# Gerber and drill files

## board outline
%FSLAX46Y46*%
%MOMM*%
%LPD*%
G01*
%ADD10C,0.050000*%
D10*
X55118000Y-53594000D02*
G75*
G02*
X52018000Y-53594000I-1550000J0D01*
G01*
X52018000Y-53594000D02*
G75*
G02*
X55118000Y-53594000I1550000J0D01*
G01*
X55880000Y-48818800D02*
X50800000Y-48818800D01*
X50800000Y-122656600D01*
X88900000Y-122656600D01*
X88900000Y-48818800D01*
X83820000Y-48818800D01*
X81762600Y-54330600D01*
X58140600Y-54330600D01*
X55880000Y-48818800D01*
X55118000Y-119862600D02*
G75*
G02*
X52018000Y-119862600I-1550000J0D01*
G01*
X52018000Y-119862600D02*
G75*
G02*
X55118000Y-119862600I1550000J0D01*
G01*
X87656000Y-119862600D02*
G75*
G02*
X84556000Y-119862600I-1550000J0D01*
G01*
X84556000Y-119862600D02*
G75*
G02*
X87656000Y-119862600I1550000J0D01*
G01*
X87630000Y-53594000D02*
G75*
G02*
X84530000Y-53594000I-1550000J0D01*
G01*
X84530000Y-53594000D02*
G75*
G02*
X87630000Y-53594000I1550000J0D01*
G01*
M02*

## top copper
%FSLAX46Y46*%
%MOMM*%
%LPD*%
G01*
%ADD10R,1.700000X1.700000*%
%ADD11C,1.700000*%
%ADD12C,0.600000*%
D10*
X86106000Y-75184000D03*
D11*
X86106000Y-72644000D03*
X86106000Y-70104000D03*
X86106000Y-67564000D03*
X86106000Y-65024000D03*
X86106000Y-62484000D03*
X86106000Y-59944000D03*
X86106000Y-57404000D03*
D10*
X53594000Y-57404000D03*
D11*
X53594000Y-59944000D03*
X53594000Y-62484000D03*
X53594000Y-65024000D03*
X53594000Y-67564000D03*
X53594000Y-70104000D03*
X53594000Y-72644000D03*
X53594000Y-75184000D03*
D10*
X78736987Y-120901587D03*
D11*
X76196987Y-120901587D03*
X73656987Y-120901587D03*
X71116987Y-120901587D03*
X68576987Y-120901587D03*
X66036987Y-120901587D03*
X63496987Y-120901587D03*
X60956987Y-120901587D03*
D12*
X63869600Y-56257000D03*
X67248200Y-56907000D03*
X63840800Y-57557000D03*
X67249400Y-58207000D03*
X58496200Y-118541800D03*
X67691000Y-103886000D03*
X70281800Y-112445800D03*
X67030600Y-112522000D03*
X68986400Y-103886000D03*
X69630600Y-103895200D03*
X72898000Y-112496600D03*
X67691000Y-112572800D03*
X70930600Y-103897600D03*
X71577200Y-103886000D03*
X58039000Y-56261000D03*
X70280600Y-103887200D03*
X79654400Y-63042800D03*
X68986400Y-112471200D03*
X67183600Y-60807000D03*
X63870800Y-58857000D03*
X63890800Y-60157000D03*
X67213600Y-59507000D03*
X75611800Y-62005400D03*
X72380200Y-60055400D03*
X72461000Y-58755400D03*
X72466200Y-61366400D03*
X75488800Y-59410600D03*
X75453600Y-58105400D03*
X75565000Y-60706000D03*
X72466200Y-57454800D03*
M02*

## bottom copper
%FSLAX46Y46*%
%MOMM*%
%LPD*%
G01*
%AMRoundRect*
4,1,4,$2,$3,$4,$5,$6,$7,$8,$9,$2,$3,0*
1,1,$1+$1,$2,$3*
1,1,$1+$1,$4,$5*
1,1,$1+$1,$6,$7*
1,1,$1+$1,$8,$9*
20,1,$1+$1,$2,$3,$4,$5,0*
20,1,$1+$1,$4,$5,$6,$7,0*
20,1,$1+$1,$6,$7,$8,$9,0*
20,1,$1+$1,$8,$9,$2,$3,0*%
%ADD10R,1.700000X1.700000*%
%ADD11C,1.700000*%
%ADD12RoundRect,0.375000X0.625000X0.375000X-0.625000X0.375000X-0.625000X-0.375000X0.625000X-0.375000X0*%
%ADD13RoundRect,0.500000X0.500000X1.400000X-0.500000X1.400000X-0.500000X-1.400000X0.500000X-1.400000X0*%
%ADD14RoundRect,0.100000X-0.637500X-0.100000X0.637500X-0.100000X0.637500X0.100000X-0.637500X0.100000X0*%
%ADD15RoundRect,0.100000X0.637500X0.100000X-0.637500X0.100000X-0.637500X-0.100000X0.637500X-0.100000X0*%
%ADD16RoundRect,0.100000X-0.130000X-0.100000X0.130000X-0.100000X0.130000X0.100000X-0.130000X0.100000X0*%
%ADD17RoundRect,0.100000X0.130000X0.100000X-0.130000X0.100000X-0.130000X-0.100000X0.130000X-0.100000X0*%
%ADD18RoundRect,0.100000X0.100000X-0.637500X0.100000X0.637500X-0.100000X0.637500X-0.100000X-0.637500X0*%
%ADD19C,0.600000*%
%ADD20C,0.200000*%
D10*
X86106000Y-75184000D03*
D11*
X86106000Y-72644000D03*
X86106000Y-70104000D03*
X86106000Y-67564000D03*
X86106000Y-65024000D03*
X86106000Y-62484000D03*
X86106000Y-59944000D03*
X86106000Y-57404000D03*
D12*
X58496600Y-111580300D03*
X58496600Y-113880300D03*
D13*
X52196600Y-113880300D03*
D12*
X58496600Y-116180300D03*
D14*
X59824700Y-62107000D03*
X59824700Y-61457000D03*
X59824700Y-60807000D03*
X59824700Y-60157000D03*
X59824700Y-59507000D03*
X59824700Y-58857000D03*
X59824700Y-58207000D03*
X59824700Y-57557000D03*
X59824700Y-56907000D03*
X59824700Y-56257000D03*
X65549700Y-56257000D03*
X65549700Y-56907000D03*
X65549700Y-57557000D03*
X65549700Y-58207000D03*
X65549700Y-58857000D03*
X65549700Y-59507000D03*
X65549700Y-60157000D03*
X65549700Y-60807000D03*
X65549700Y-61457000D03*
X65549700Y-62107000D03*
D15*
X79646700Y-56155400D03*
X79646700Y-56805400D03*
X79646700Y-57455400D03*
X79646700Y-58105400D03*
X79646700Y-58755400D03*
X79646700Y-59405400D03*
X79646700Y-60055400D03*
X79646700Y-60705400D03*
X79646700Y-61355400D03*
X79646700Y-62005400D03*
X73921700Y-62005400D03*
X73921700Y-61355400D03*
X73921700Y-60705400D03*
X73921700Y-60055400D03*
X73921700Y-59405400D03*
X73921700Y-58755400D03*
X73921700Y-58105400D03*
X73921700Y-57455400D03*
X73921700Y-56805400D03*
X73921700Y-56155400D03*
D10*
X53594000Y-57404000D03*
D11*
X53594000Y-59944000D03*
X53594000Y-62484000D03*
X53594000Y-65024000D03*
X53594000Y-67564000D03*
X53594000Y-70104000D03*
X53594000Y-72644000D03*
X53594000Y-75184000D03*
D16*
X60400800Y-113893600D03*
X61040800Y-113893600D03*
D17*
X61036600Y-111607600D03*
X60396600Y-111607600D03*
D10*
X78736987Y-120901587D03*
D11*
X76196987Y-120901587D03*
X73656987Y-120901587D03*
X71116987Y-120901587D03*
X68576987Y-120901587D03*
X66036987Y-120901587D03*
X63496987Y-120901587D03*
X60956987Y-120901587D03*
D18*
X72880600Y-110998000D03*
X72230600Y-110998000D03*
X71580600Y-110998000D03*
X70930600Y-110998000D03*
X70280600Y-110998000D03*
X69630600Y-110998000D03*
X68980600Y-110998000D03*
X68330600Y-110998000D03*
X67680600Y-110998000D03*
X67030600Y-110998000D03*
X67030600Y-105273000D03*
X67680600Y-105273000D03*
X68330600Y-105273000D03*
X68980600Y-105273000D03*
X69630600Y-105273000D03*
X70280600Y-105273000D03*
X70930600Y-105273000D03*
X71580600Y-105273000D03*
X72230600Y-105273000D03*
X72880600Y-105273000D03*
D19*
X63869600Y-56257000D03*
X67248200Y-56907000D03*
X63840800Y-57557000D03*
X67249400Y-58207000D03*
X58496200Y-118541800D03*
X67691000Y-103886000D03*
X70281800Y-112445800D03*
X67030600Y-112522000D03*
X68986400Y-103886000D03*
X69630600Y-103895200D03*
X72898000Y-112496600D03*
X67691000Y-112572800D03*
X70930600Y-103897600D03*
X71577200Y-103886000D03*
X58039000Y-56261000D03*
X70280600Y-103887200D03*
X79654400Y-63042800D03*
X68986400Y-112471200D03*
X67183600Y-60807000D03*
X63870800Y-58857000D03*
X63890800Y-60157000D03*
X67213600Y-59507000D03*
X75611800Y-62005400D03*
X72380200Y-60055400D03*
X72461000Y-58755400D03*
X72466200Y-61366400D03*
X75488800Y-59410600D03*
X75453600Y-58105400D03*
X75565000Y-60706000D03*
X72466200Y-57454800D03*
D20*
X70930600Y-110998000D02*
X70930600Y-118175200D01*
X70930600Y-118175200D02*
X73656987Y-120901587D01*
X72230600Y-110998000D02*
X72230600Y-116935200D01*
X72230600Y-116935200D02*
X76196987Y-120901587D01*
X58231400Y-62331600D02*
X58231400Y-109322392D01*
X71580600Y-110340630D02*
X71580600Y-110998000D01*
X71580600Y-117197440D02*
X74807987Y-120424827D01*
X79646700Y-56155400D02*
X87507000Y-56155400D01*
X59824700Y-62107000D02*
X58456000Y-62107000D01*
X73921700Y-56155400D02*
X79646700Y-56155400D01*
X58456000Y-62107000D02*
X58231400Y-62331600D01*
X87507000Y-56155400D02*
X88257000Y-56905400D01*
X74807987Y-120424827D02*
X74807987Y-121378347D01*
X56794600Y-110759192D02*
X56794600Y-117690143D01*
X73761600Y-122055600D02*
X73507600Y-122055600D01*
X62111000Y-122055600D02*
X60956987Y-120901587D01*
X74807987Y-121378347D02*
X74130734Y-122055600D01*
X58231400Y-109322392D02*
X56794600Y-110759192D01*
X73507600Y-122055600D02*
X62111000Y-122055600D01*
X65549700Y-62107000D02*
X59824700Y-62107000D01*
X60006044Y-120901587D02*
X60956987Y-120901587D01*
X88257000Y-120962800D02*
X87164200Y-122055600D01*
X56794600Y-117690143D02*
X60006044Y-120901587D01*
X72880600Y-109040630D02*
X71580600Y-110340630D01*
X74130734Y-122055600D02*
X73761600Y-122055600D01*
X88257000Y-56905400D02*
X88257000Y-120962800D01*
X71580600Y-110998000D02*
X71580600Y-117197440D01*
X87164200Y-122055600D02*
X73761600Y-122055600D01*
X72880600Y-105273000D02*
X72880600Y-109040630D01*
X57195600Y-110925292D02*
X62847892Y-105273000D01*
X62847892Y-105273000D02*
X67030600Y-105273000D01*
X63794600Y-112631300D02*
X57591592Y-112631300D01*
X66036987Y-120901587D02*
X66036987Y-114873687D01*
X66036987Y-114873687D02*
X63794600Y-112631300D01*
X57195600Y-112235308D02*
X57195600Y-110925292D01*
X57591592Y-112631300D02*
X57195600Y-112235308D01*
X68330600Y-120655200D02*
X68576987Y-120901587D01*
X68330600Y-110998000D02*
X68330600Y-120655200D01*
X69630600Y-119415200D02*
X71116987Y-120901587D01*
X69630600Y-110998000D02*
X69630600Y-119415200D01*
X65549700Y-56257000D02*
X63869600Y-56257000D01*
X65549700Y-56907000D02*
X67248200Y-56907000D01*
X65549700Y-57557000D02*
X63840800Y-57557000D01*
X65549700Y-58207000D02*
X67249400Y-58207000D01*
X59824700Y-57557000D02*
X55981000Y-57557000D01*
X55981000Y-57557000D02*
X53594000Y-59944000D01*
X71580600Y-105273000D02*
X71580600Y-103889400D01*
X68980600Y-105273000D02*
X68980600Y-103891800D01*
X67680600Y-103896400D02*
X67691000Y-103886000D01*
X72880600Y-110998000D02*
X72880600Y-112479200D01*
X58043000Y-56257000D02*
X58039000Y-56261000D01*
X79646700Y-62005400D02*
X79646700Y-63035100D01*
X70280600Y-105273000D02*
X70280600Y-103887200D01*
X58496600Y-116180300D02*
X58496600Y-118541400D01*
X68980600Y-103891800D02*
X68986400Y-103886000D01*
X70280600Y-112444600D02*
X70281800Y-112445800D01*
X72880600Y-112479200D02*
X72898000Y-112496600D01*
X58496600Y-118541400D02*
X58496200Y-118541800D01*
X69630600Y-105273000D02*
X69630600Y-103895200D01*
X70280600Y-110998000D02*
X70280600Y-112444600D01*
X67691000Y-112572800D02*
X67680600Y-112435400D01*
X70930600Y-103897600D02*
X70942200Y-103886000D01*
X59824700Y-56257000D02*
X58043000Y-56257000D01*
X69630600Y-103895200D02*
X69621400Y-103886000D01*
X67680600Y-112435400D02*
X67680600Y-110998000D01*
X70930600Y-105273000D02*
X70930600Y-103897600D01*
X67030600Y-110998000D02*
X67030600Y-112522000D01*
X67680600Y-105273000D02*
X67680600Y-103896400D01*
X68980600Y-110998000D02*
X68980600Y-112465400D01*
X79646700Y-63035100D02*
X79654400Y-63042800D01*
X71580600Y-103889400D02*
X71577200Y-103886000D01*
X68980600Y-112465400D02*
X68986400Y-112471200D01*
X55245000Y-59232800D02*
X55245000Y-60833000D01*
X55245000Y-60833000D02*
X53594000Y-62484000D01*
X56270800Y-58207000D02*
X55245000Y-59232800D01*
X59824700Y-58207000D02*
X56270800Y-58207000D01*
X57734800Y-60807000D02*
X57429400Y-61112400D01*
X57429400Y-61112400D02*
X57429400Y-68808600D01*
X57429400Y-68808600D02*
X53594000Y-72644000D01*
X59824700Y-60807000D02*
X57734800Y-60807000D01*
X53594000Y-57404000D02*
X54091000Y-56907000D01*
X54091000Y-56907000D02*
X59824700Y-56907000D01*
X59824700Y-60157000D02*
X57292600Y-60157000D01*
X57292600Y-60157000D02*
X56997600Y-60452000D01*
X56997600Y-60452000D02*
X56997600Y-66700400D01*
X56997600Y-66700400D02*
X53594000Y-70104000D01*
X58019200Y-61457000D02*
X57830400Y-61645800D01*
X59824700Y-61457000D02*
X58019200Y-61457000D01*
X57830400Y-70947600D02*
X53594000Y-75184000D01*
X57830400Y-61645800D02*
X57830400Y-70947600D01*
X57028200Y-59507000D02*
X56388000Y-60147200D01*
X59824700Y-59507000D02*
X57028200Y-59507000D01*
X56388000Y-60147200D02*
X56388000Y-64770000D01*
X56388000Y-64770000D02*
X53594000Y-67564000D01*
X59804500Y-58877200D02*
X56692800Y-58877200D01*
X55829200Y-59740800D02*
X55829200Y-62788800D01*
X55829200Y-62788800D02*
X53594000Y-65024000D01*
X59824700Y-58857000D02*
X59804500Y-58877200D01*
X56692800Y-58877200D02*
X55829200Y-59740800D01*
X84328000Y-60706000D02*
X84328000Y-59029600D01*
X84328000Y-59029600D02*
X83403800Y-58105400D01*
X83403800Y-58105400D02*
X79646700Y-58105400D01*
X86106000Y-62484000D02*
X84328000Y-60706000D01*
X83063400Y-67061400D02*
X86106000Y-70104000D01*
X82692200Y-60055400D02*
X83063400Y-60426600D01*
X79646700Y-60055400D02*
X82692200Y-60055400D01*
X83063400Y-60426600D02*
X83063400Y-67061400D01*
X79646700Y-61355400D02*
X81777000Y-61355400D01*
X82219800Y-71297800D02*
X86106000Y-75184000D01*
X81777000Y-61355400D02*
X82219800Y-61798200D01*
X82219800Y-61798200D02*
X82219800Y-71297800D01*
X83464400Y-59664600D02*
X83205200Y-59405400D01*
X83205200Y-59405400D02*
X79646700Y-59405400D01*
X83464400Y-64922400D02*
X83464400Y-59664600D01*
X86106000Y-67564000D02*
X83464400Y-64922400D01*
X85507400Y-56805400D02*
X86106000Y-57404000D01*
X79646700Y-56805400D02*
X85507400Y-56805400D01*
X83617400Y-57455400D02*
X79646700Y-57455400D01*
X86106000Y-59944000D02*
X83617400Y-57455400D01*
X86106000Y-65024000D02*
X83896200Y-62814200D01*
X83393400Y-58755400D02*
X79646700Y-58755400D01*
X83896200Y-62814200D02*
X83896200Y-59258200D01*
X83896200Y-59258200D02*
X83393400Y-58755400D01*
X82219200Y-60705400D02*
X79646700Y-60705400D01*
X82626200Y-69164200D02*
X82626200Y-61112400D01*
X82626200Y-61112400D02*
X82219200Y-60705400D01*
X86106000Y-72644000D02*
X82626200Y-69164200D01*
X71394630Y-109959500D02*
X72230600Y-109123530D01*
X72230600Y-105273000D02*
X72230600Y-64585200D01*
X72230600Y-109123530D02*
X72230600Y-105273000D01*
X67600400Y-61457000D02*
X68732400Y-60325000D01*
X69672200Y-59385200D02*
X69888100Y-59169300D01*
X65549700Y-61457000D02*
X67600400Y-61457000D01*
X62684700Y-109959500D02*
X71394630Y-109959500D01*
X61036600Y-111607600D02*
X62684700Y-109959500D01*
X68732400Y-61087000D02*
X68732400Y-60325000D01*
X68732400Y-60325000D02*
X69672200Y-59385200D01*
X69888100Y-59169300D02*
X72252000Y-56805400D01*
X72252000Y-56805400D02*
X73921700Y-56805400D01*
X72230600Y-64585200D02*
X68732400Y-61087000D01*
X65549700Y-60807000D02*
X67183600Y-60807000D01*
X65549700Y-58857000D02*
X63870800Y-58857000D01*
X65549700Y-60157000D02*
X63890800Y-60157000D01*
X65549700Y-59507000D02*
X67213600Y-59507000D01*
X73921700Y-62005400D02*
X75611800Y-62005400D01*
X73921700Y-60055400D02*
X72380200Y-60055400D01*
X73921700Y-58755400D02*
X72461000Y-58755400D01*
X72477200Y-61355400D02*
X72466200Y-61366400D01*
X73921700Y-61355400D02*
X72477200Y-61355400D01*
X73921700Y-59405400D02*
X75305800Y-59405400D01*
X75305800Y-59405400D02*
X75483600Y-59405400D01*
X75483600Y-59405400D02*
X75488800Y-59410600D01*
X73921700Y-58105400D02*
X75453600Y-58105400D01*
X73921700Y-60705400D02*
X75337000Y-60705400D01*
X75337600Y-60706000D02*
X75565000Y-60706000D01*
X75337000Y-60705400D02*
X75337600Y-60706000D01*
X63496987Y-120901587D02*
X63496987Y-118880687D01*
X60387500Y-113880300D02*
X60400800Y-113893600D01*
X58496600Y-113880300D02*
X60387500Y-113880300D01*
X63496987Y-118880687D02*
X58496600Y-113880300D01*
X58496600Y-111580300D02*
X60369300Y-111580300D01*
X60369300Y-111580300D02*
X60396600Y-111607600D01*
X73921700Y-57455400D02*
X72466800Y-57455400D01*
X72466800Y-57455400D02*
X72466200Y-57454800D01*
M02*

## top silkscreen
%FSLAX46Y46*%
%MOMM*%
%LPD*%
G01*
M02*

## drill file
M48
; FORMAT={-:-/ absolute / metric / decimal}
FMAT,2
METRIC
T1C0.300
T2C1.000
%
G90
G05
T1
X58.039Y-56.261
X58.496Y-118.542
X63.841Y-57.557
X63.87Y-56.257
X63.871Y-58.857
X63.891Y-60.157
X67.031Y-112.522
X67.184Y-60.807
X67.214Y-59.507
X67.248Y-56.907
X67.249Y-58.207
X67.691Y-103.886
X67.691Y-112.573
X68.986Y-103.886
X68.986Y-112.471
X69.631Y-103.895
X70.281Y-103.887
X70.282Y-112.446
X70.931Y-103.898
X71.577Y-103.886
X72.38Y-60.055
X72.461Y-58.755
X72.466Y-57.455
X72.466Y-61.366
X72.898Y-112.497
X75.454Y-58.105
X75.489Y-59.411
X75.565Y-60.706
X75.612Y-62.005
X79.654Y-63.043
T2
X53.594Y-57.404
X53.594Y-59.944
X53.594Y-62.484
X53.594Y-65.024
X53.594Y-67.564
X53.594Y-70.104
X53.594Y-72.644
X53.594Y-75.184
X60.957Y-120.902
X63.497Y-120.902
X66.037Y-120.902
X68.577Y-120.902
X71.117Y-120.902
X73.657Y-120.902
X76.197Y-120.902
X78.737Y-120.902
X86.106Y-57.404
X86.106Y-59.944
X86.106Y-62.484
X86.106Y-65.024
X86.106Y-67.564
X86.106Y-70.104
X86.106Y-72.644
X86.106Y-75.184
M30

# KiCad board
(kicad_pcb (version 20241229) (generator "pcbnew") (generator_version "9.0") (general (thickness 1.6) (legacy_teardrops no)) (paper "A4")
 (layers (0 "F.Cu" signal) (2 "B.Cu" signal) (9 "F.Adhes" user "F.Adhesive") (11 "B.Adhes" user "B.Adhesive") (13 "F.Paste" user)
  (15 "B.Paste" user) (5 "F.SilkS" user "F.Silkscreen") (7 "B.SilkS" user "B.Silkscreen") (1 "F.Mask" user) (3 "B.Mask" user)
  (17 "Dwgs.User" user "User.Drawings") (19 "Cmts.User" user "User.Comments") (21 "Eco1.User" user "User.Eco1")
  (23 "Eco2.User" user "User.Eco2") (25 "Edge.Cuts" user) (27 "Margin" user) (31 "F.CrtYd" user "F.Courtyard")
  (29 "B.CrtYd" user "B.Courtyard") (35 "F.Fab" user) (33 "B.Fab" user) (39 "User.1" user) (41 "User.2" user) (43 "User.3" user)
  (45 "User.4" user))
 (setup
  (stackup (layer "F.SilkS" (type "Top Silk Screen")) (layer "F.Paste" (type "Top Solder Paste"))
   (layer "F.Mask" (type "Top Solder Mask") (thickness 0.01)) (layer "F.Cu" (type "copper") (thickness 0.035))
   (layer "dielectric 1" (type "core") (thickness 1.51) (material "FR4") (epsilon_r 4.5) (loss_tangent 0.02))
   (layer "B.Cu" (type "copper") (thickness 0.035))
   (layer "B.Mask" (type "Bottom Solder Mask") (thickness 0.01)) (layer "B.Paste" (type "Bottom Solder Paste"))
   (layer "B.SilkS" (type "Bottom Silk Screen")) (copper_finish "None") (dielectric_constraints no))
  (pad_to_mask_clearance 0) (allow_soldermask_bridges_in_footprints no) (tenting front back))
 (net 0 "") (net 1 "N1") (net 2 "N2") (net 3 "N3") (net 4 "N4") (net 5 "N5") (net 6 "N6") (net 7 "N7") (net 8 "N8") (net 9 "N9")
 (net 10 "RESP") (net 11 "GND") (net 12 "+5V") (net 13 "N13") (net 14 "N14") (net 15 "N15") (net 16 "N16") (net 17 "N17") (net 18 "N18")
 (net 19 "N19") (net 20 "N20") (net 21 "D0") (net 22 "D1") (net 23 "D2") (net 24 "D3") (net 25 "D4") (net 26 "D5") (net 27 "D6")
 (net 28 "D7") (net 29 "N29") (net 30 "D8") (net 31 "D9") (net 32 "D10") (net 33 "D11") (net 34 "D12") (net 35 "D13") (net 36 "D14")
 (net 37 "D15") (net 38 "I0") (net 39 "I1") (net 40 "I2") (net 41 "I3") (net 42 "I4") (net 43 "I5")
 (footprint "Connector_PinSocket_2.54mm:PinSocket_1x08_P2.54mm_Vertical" (layer "B.Cu") (at 86.106 75.184)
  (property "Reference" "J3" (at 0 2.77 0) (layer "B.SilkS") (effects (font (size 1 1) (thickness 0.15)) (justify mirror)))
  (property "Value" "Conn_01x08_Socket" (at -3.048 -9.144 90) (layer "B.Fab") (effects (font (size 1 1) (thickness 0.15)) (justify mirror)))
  (pad "1" thru_hole rect (at 0 0) (size 1.7 1.7) (drill 1) (layers "*.Cu" "*.Mask") (remove_unused_layers no) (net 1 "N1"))
  (pad "2" thru_hole circle (at 0 -2.54) (size 1.7 1.7) (drill 1) (layers "*.Cu" "*.Mask") (remove_unused_layers no) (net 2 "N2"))
  (pad "3" thru_hole circle (at 0 -5.08) (size 1.7 1.7) (drill 1) (layers "*.Cu" "*.Mask") (remove_unused_layers no) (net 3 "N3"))
  (pad "4" thru_hole circle (at 0 -7.62) (size 1.7 1.7) (drill 1) (layers "*.Cu" "*.Mask") (remove_unused_layers no) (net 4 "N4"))
  (pad "5" thru_hole circle (at 0 -10.16) (size 1.7 1.7) (drill 1) (layers "*.Cu" "*.Mask") (remove_unused_layers no) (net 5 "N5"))
  (pad "6" thru_hole circle (at 0 -12.7) (size 1.7 1.7) (drill 1) (layers "*.Cu" "*.Mask") (remove_unused_layers no) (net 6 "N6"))
  (pad "7" thru_hole circle (at 0 -15.24) (size 1.7 1.7) (drill 1) (layers "*.Cu" "*.Mask") (remove_unused_layers no) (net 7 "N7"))
  (pad "8" thru_hole circle (at 0 -17.78) (size 1.7 1.7) (drill 1) (layers "*.Cu" "*.Mask") (remove_unused_layers no) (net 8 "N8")))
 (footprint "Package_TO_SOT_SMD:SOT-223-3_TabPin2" (layer "B.Cu") (at 55.3466 113.8803 180)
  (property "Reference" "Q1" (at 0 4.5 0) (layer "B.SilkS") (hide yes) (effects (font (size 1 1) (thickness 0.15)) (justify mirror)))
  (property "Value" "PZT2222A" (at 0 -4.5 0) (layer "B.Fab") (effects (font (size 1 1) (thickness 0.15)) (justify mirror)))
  (pad "1" smd roundrect (at -3.15 2.3 180) (size 2 1.5) (layers "B.Cu" "B.Mask" "B.Paste") (roundrect_rratio 0.25) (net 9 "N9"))
  (pad "2" smd roundrect (at -3.15 0 180) (size 2 1.5) (layers "B.Cu" "B.Mask" "B.Paste") (roundrect_rratio 0.25) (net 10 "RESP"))
  (pad "2" smd roundrect (at 3.15 0 180) (size 2 3.8) (layers "B.Cu" "B.Mask" "B.Paste") (roundrect_rratio 0.25) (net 10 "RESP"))
  (pad "3" smd roundrect (at -3.15 -2.3 180) (size 2 1.5) (layers "B.Cu" "B.Mask" "B.Paste") (roundrect_rratio 0.25) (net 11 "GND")))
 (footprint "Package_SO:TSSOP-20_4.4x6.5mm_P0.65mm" (layer "B.Cu") (at 62.6872 59.182)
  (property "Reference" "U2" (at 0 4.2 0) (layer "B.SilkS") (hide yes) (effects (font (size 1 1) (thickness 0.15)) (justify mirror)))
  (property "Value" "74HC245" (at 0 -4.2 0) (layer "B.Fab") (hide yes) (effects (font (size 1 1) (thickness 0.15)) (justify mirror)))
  (pad "1" smd roundrect (at -2.8625 2.925) (size 1.475 0.4) (layers "B.Cu" "B.Mask" "B.Paste") (roundrect_rratio 0.25) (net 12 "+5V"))
  (pad "2" smd roundrect (at -2.8625 2.275) (size 1.475 0.4) (layers "B.Cu" "B.Mask" "B.Paste") (roundrect_rratio 0.25) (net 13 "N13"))
  (pad "3" smd roundrect (at -2.8625 1.625) (size 1.475 0.4) (layers "B.Cu" "B.Mask" "B.Paste") (roundrect_rratio 0.25) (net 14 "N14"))
  (pad "4" smd roundrect (at -2.8625 0.975) (size 1.475 0.4) (layers "B.Cu" "B.Mask" "B.Paste") (roundrect_rratio 0.25) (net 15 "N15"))
  (pad "5" smd roundrect (at -2.8625 0.325) (size 1.475 0.4) (layers "B.Cu" "B.Mask" "B.Paste") (roundrect_rratio 0.25) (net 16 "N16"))
  (pad "6" smd roundrect (at -2.8625 -0.325) (size 1.475 0.4) (layers "B.Cu" "B.Mask" "B.Paste") (roundrect_rratio 0.25) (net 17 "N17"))
  (pad "7" smd roundrect (at -2.8625 -0.975) (size 1.475 0.4) (layers "B.Cu" "B.Mask" "B.Paste") (roundrect_rratio 0.25) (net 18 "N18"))
  (pad "8" smd roundrect (at -2.8625 -1.625) (size 1.475 0.4) (layers "B.Cu" "B.Mask" "B.Paste") (roundrect_rratio 0.25) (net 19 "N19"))
  (pad "9" smd roundrect (at -2.8625 -2.275) (size 1.475 0.4) (layers "B.Cu" "B.Mask" "B.Paste") (roundrect_rratio 0.25) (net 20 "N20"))
  (pad "10" smd roundrect (at -2.8625 -2.925) (size 1.475 0.4) (layers "B.Cu" "B.Mask" "B.Paste") (roundrect_rratio 0.25) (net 11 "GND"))
  (pad "11" smd roundrect (at 2.8625 -2.925) (size 1.475 0.4) (layers "B.Cu" "B.Mask" "B.Paste") (roundrect_rratio 0.25) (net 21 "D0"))
  (pad "12" smd roundrect (at 2.8625 -2.275) (size 1.475 0.4) (layers "B.Cu" "B.Mask" "B.Paste") (roundrect_rratio 0.25) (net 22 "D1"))
  (pad "13" smd roundrect (at 2.8625 -1.625) (size 1.475 0.4) (layers "B.Cu" "B.Mask" "B.Paste") (roundrect_rratio 0.25) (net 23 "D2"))
  (pad "14" smd roundrect (at 2.8625 -0.975) (size 1.475 0.4) (layers "B.Cu" "B.Mask" "B.Paste") (roundrect_rratio 0.25) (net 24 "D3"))
  (pad "15" smd roundrect (at 2.8625 -0.325) (size 1.475 0.4) (layers "B.Cu" "B.Mask" "B.Paste") (roundrect_rratio 0.25) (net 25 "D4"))
  (pad "16" smd roundrect (at 2.8625 0.325) (size 1.475 0.4) (layers "B.Cu" "B.Mask" "B.Paste") (roundrect_rratio 0.25) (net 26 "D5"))
  (pad "17" smd roundrect (at 2.8625 0.975) (size 1.475 0.4) (layers "B.Cu" "B.Mask" "B.Paste") (roundrect_rratio 0.25) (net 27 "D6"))
  (pad "18" smd roundrect (at 2.8625 1.625) (size 1.475 0.4) (layers "B.Cu" "B.Mask" "B.Paste") (roundrect_rratio 0.25) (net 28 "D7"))
  (pad "19" smd roundrect (at 2.8625 2.275) (size 1.475 0.4) (layers "B.Cu" "B.Mask" "B.Paste") (roundrect_rratio 0.25) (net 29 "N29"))
  (pad "20" smd roundrect (at 2.8625 2.925) (size 1.475 0.4) (layers "B.Cu" "B.Mask" "B.Paste") (roundrect_rratio 0.25) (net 12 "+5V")))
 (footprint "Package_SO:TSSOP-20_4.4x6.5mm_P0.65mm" (layer "B.Cu") (at 76.7842 59.0804 180)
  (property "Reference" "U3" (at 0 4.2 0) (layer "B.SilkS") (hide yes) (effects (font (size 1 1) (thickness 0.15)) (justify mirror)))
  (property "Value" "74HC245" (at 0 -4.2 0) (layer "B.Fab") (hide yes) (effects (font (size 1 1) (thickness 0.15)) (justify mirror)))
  (pad "1" smd roundrect (at -2.8625 2.925 180) (size 1.475 0.4) (layers "B.Cu" "B.Mask" "B.Paste") (roundrect_rratio 0.25) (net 12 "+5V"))
  (pad "2" smd roundrect (at -2.8625 2.275 180) (size 1.475 0.4) (layers "B.Cu" "B.Mask" "B.Paste") (roundrect_rratio 0.25) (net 8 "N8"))
  (pad "3" smd roundrect (at -2.8625 1.625 180) (size 1.475 0.4) (layers "B.Cu" "B.Mask" "B.Paste") (roundrect_rratio 0.25) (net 7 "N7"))
  (pad "4" smd roundrect (at -2.8625 0.975 180) (size 1.475 0.4) (layers "B.Cu" "B.Mask" "B.Paste") (roundrect_rratio 0.25) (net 6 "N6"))
  (pad "5" smd roundrect (at -2.8625 0.325 180) (size 1.475 0.4) (layers "B.Cu" "B.Mask" "B.Paste") (roundrect_rratio 0.25) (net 5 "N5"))
  (pad "6" smd roundrect (at -2.8625 -0.325 180) (size 1.475 0.4) (layers "B.Cu" "B.Mask" "B.Paste") (roundrect_rratio 0.25) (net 4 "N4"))
  (pad "7" smd roundrect (at -2.8625 -0.975 180) (size 1.475 0.4) (layers "B.Cu" "B.Mask" "B.Paste") (roundrect_rratio 0.25) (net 3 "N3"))
  (pad "8" smd roundrect (at -2.8625 -1.625 180) (size 1.475 0.4) (layers "B.Cu" "B.Mask" "B.Paste") (roundrect_rratio 0.25) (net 2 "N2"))
  (pad "9" smd roundrect (at -2.8625 -2.275 180) (size 1.475 0.4) (layers "B.Cu" "B.Mask" "B.Paste") (roundrect_rratio 0.25) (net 1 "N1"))
  (pad "10" smd roundrect (at -2.8625 -2.925 180) (size 1.475 0.4) (layers "B.Cu" "B.Mask" "B.Paste") (roundrect_rratio 0.25) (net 11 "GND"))
  (pad "11" smd roundrect (at 2.8625 -2.925 180) (size 1.475 0.4) (layers "B.Cu" "B.Mask" "B.Paste") (roundrect_rratio 0.25) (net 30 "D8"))
  (pad "12" smd roundrect (at 2.8625 -2.275 180) (size 1.475 0.4) (layers "B.Cu" "B.Mask" "B.Paste") (roundrect_rratio 0.25) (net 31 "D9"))
  (pad "13" smd roundrect (at 2.8625 -1.625 180) (size 1.475 0.4) (layers "B.Cu" "B.Mask" "B.Paste") (roundrect_rratio 0.25) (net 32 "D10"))
  (pad "14" smd roundrect (at 2.8625 -0.975 180) (size 1.475 0.4) (layers "B.Cu" "B.Mask" "B.Paste") (roundrect_rratio 0.25) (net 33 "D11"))
  (pad "15" smd roundrect (at 2.8625 -0.325 180) (size 1.475 0.4) (layers "B.Cu" "B.Mask" "B.Paste") (roundrect_rratio 0.25) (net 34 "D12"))
  (pad "16" smd roundrect (at 2.8625 0.325 180) (size 1.475 0.4) (layers "B.Cu" "B.Mask" "B.Paste") (roundrect_rratio 0.25) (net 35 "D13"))
  (pad "17" smd roundrect (at 2.8625 0.975 180) (size 1.475 0.4) (layers "B.Cu" "B.Mask" "B.Paste") (roundrect_rratio 0.25) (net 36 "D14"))
  (pad "18" smd roundrect (at 2.8625 1.625 180) (size 1.475 0.4) (layers "B.Cu" "B.Mask" "B.Paste") (roundrect_rratio 0.25) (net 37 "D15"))
  (pad "19" smd roundrect (at 2.8625 2.275 180) (size 1.475 0.4) (layers "B.Cu" "B.Mask" "B.Paste") (roundrect_rratio 0.25) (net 29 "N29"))
  (pad "20" smd roundrect (at 2.8625 2.925 180) (size 1.475 0.4) (layers "B.Cu" "B.Mask" "B.Paste") (roundrect_rratio 0.25) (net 12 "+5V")))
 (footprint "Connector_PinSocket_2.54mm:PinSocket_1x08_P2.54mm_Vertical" (layer "B.Cu") (at 53.594 57.404 180)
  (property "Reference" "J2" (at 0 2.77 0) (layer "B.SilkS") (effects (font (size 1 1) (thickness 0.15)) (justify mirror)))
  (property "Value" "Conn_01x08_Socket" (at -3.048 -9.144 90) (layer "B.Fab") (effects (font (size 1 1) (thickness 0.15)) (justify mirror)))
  (pad "1" thru_hole rect (at 0 0 180) (size 1.7 1.7) (drill 1) (layers "*.Cu" "*.Mask") (remove_unused_layers no) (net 20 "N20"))
  (pad "2" thru_hole circle (at 0 -2.54 180) (size 1.7 1.7) (drill 1) (layers "*.Cu" "*.Mask") (remove_unused_layers no) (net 19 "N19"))
  (pad "3" thru_hole circle (at 0 -5.08 180) (size 1.7 1.7) (drill 1) (layers "*.Cu" "*.Mask") (remove_unused_layers no) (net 18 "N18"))
  (pad "4" thru_hole circle (at 0 -7.62 180) (size 1.7 1.7) (drill 1) (layers "*.Cu" "*.Mask") (remove_unused_layers no) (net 17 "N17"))
  (pad "5" thru_hole circle (at 0 -10.16 180) (size 1.7 1.7) (drill 1) (layers "*.Cu" "*.Mask") (remove_unused_layers no) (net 16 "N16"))
  (pad "6" thru_hole circle (at 0 -12.7 180) (size 1.7 1.7) (drill 1) (layers "*.Cu" "*.Mask") (remove_unused_layers no) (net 15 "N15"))
  (pad "7" thru_hole circle (at 0 -15.24 180) (size 1.7 1.7) (drill 1) (layers "*.Cu" "*.Mask") (remove_unused_layers no) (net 14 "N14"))
  (pad "8" thru_hole circle (at 0 -17.78 180) (size 1.7 1.7) (drill 1) (layers "*.Cu" "*.Mask") (remove_unused_layers no) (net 13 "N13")))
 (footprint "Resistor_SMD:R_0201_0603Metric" (layer "B.Cu") (at 60.7208 113.8936)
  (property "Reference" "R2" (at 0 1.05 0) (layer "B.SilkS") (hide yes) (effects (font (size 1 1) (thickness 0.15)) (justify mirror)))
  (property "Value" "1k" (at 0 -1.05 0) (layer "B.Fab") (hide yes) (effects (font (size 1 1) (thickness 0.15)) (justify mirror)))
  (pad "" smd roundrect (at -0.345 0) (size 0.318 0.36) (layers "B.Paste") (roundrect_rratio 0.25))
  (pad "" smd roundrect (at 0.345 0) (size 0.318 0.36) (layers "B.Paste") (roundrect_rratio 0.25))
  (pad "1" smd roundrect (at -0.32 0) (size 0.46 0.4) (layers "B.Cu" "B.Mask") (roundrect_rratio 0.25) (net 10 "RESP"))
  (pad "2" smd roundrect (at 0.32 0) (size 0.46 0.4) (layers "B.Cu" "B.Mask") (roundrect_rratio 0.25) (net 12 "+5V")))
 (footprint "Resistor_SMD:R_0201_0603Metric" (layer "B.Cu") (at 60.7166 111.6076 180)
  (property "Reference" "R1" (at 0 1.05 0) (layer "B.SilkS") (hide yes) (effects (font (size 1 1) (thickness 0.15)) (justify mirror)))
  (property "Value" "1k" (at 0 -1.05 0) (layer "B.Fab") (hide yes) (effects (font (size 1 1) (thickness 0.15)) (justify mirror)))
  (pad "" smd roundrect (at -0.345 0 180) (size 0.318 0.36) (layers "B.Paste") (roundrect_rratio 0.25))
  (pad "" smd roundrect (at 0.345 0 180) (size 0.318 0.36) (layers "B.Paste") (roundrect_rratio 0.25))
  (pad "1" smd roundrect (at -0.32 0 180) (size 0.46 0.4) (layers "B.Cu" "B.Mask") (roundrect_rratio 0.25) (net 29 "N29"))
  (pad "2" smd roundrect (at 0.32 0 180) (size 0.46 0.4) (layers "B.Cu" "B.Mask") (roundrect_rratio 0.25) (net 9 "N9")))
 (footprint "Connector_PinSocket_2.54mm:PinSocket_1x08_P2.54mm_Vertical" (layer "B.Cu") (at 78.736987 120.901587 90)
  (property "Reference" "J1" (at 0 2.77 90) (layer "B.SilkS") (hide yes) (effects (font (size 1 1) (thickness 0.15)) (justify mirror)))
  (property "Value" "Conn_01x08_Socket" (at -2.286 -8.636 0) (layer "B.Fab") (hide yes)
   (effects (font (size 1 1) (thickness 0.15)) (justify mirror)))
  (pad "1" thru_hole rect (at 0 0 90) (size 1.7 1.7) (drill 1) (layers "*.Cu" "*.Mask") (remove_unused_layers no) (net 11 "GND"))
  (pad "2" thru_hole circle (at 0 -2.54 90) (size 1.7 1.7) (drill 1) (layers "*.Cu" "*.Mask") (remove_unused_layers no) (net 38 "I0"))
  (pad "3" thru_hole circle (at 0 -5.08 90) (size 1.7 1.7) (drill 1) (layers "*.Cu" "*.Mask") (remove_unused_layers no) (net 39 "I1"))
  (pad "4" thru_hole circle (at 0 -7.62 90) (size 1.7 1.7) (drill 1) (layers "*.Cu" "*.Mask") (remove_unused_layers no) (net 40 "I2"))
  (pad "5" thru_hole circle (at 0 -10.16 90) (size 1.7 1.7) (drill 1) (layers "*.Cu" "*.Mask") (remove_unused_layers no) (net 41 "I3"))
  (pad "6" thru_hole circle (at 0 -12.7 90) (size 1.7 1.7) (drill 1) (layers "*.Cu" "*.Mask") (remove_unused_layers no) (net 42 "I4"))
  (pad "7" thru_hole circle (at 0 -15.24 90) (size 1.7 1.7) (drill 1) (layers "*.Cu" "*.Mask") (remove_unused_layers no) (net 10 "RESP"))
  (pad "8" thru_hole circle (at 0 -17.78 90) (size 1.7 1.7) (drill 1) (layers "*.Cu" "*.Mask") (remove_unused_layers no) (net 12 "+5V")))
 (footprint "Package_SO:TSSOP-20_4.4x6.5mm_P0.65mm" (layer "B.Cu") (at 69.9556 108.1355 90)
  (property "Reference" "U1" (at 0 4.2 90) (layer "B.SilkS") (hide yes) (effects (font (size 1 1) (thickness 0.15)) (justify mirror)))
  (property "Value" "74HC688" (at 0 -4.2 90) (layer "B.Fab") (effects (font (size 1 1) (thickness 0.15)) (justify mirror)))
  (pad "1" smd roundrect (at -2.8625 2.925 90) (size 1.475 0.4) (layers "B.Cu" "B.Mask" "B.Paste") (roundrect_rratio 0.25) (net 11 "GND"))
  (pad "2" smd roundrect (at -2.8625 2.275 90) (size 1.475 0.4) (layers "B.Cu" "B.Mask" "B.Paste") (roundrect_rratio 0.25) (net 38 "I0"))
  (pad "3" smd roundrect (at -2.8625 1.625 90) (size 1.475 0.4) (layers "B.Cu" "B.Mask" "B.Paste") (roundrect_rratio 0.25) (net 12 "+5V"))
  (pad "4" smd roundrect (at -2.8625 0.975 90) (size 1.475 0.4) (layers "B.Cu" "B.Mask" "B.Paste") (roundrect_rratio 0.25) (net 39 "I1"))
  (pad "5" smd roundrect (at -2.8625 0.325 90) (size 1.475 0.4) (layers "B.Cu" "B.Mask" "B.Paste") (roundrect_rratio 0.25) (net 11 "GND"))
  (pad "6" smd roundrect (at -2.8625 -0.325 90) (size 1.475 0.4) (layers "B.Cu" "B.Mask" "B.Paste") (roundrect_rratio 0.25) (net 40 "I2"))
  (pad "7" smd roundrect (at -2.8625 -0.975 90) (size 1.475 0.4) (layers "B.Cu" "B.Mask" "B.Paste") (roundrect_rratio 0.25) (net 11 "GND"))
  (pad "8" smd roundrect (at -2.8625 -1.625 90) (size 1.475 0.4) (layers "B.Cu" "B.Mask" "B.Paste") (roundrect_rratio 0.25) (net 41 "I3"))
  (pad "9" smd roundrect (at -2.8625 -2.275 90) (size 1.475 0.4) (layers "B.Cu" "B.Mask" "B.Paste") (roundrect_rratio 0.25) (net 11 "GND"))
  (pad "10" smd roundrect (at -2.8625 -2.925 90) (size 1.475 0.4) (layers "B.Cu" "B.Mask" "B.Paste") (roundrect_rratio 0.25) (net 11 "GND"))
  (pad "11" smd roundrect (at 2.8625 -2.925 90) (size 1.475 0.4) (layers "B.Cu" "B.Mask" "B.Paste") (roundrect_rratio 0.25) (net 42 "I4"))
  (pad "12" smd roundrect (at 2.8625 -2.275 90) (size 1.475 0.4) (layers "B.Cu" "B.Mask" "B.Paste") (roundrect_rratio 0.25) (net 11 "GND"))
  (pad "13" smd roundrect (at 2.8625 -1.625 90) (size 1.475 0.4) (layers "B.Cu" "B.Mask" "B.Paste") (roundrect_rratio 0.25) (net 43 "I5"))
  (pad "14" smd roundrect (at 2.8625 -0.975 90) (size 1.475 0.4) (layers "B.Cu" "B.Mask" "B.Paste") (roundrect_rratio 0.25) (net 11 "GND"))
  (pad "15" smd roundrect (at 2.8625 -0.325 90) (size 1.475 0.4) (layers "B.Cu" "B.Mask" "B.Paste") (roundrect_rratio 0.25) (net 11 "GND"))
  (pad "16" smd roundrect (at 2.8625 0.325 90) (size 1.475 0.4) (layers "B.Cu" "B.Mask" "B.Paste") (roundrect_rratio 0.25) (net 11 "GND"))
  (pad "17" smd roundrect (at 2.8625 0.975 90) (size 1.475 0.4) (layers "B.Cu" "B.Mask" "B.Paste") (roundrect_rratio 0.25) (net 11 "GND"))
  (pad "18" smd roundrect (at 2.8625 1.625 90) (size 1.475 0.4) (layers "B.Cu" "B.Mask" "B.Paste") (roundrect_rratio 0.25) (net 11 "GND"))
  (pad "19" smd roundrect (at 2.8625 2.275 90) (size 1.475 0.4) (layers "B.Cu" "B.Mask" "B.Paste") (roundrect_rratio 0.25) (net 29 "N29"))
  (pad "20" smd roundrect (at 2.8625 2.925 90) (size 1.475 0.4) (layers "B.Cu" "B.Mask" "B.Paste") (roundrect_rratio 0.25) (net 12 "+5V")))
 (gr_circle (center 53.568 53.594) (end 55.118 53.594) (stroke (width 0.05) (type solid)) (fill no) (layer "Edge.Cuts"))
 (gr_poly
  (pts (xy 55.88 48.8188) (xy 50.8 48.8188) (xy 50.8 122.6566) (xy 88.9 122.6566) (xy 88.9 48.8188) (xy 83.82 48.8188) (xy 81.7626 54.3306)
   (xy 58.1406 54.3306))
  (stroke (width 0.05) (type solid)) (fill no) (layer "Edge.Cuts"))
 (gr_circle (center 53.568 119.8626) (end 55.118 119.8626) (stroke (width 0.05) (type solid)) (fill no) (layer "Edge.Cuts"))
 (gr_circle (center 86.106 119.8626) (end 87.656 119.8626) (stroke (width 0.05) (type solid)) (fill no) (layer "Edge.Cuts"))
 (gr_circle (center 86.08 53.594) (end 87.63 53.594) (stroke (width 0.05) (type solid)) (fill no) (layer "Edge.Cuts"))
 (segment (start 70.9306 110.998) (end 70.9306 118.1752) (width 0.2) (layer "B.Cu") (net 39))
 (segment (start 70.9306 118.1752) (end 73.656987 120.901587) (width 0.2) (layer "B.Cu") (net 39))
 (segment (start 72.2306 110.998) (end 72.2306 116.9352) (width 0.2) (layer "B.Cu") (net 38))
 (segment (start 72.2306 116.9352) (end 76.196987 120.901587) (width 0.2) (layer "B.Cu") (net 38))
 (segment (start 58.2314 62.3316) (end 58.2314 109.322392) (width 0.2) (layer "B.Cu") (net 12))
 (segment (start 71.5806 110.34063) (end 71.5806 110.998) (width 0.2) (layer "B.Cu") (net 12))
 (segment (start 71.5806 117.19744) (end 74.807987 120.424827) (width 0.2) (layer "B.Cu") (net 12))
 (segment (start 79.6467 56.1554) (end 87.507 56.1554) (width 0.2) (layer "B.Cu") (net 12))
 (segment (start 59.8247 62.107) (end 58.456 62.107) (width 0.2) (layer "B.Cu") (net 12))
 (segment (start 73.9217 56.1554) (end 79.6467 56.1554) (width 0.2) (layer "B.Cu") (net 12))
 (segment (start 58.456 62.107) (end 58.2314 62.3316) (width 0.2) (layer "B.Cu") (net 12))
 (segment (start 87.507 56.1554) (end 88.257 56.9054) (width 0.2) (layer "B.Cu") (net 12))
 (segment (start 74.807987 120.424827) (end 74.807987 121.378347) (width 0.2) (layer "B.Cu") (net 12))
 (segment (start 56.7946 110.759192) (end 56.7946 117.690143) (width 0.2) (layer "B.Cu") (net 12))
 (segment (start 73.7616 122.0556) (end 73.5076 122.0556) (width 0.2) (layer "B.Cu") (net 12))
 (segment (start 62.111 122.0556) (end 60.956987 120.901587) (width 0.2) (layer "B.Cu") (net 12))
 (segment (start 74.807987 121.378347) (end 74.130734 122.0556) (width 0.2) (layer "B.Cu") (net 12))
 (segment (start 58.2314 109.322392) (end 56.7946 110.759192) (width 0.2) (layer "B.Cu") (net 12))
 (segment (start 73.5076 122.0556) (end 62.111 122.0556) (width 0.2) (layer "B.Cu") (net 12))
 (segment (start 65.5497 62.107) (end 59.8247 62.107) (width 0.2) (layer "B.Cu") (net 12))
 (segment (start 60.006044 120.901587) (end 60.956987 120.901587) (width 0.2) (layer "B.Cu") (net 12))
 (segment (start 88.257 120.9628) (end 87.1642 122.0556) (width 0.2) (layer "B.Cu") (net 12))
 (segment (start 56.7946 117.690143) (end 60.006044 120.901587) (width 0.2) (layer "B.Cu") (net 12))
 (segment (start 72.8806 109.04063) (end 71.5806 110.34063) (width 0.2) (layer "B.Cu") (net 12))
 (segment (start 74.130734 122.0556) (end 73.7616 122.0556) (width 0.2) (layer "B.Cu") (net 12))
 (segment (start 88.257 56.9054) (end 88.257 120.9628) (width 0.2) (layer "B.Cu") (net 12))
 (segment (start 71.5806 110.998) (end 71.5806 117.19744) (width 0.2) (layer "B.Cu") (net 12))
 (segment (start 87.1642 122.0556) (end 73.7616 122.0556) (width 0.2) (layer "B.Cu") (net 12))
 (segment (start 72.8806 105.273) (end 72.8806 109.04063) (width 0.2) (layer "B.Cu") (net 12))
 (segment (start 57.1956 110.925292) (end 62.847892 105.273) (width 0.2) (layer "B.Cu") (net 42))
 (segment (start 62.847892 105.273) (end 67.0306 105.273) (width 0.2) (layer "B.Cu") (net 42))
 (segment (start 63.7946 112.6313) (end 57.591592 112.6313) (width 0.2) (layer "B.Cu") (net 42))
 (segment (start 66.036987 120.901587) (end 66.036987 114.873687) (width 0.2) (layer "B.Cu") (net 42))
 (segment (start 66.036987 114.873687) (end 63.7946 112.6313) (width 0.2) (layer "B.Cu") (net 42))
 (segment (start 57.1956 112.235308) (end 57.1956 110.925292) (width 0.2) (layer "B.Cu") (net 42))
 (segment (start 57.591592 112.6313) (end 57.1956 112.235308) (width 0.2) (layer "B.Cu") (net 42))
 (segment (start 68.3306 120.6552) (end 68.576987 120.901587) (width 0.2) (layer "B.Cu") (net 41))
 (segment (start 68.3306 110.998) (end 68.3306 120.6552) (width 0.2) (layer "B.Cu") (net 41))
 (segment (start 69.6306 119.4152) (end 71.116987 120.901587) (width 0.2) (layer "B.Cu") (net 40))
 (segment (start 69.6306 110.998) (end 69.6306 119.4152) (width 0.2) (layer "B.Cu") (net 40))
 (via (at 63.8696 56.257) (size 0.6) (drill 0.3) (layers "F.Cu" "B.Cu") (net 21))
 (segment (start 65.5497 56.257) (end 63.8696 56.257) (width 0.2) (layer "B.Cu") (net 21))
 (via (at 67.2482 56.907) (size 0.6) (drill 0.3) (layers "F.Cu" "B.Cu") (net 22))
 (segment (start 65.5497 56.907) (end 67.2482 56.907) (width 0.2) (layer "B.Cu") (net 22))
 (via (at 63.8408 57.557) (size 0.6) (drill 0.3) (layers "F.Cu" "B.Cu") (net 23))
 (segment (start 65.5497 57.557) (end 63.8408 57.557) (width 0.2) (layer "B.Cu") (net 23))
 (via (at 67.2494 58.207) (size 0.6) (drill 0.3) (layers "F.Cu" "B.Cu") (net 24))
 (segment (start 65.5497 58.207) (end 67.2494 58.207) (width 0.2) (layer "B.Cu") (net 24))
 (segment (start 59.8247 57.557) (end 55.981 57.557) (width 0.2) (layer "B.Cu") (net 19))
 (segment (start 55.981 57.557) (end 53.594 59.944) (width 0.2) (layer "B.Cu") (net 19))
 (via (at 58.4962 118.5418) (size 0.6) (drill 0.3) (layers "F.Cu" "B.Cu") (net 11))
 (via (at 67.691 103.886) (size 0.6) (drill 0.3) (layers "F.Cu" "B.Cu") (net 11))
 (via (at 70.2818 112.4458) (size 0.6) (drill 0.3) (layers "F.Cu" "B.Cu") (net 11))
 (via (at 67.0306 112.522) (size 0.6) (drill 0.3) (layers "F.Cu" "B.Cu") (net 11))
 (via (at 68.9864 103.886) (size 0.6) (drill 0.3) (layers "F.Cu" "B.Cu") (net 11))
 (via (at 69.6306 103.8952) (size 0.6) (drill 0.3) (layers "F.Cu" "B.Cu") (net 11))
 (via (at 72.898 112.4966) (size 0.6) (drill 0.3) (layers "F.Cu" "B.Cu") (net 11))
 (via (at 67.691 112.5728) (size 0.6) (drill 0.3) (layers "F.Cu" "B.Cu") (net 11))
 (via (at 70.9306 103.8976) (size 0.6) (drill 0.3) (layers "F.Cu" "B.Cu") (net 11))
 (via (at 71.5772 103.886) (size 0.6) (drill 0.3) (layers "F.Cu" "B.Cu") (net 11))
 (via (at 58.039 56.261) (size 0.6) (drill 0.3) (layers "F.Cu" "B.Cu") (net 11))
 (via (at 70.2806 103.8872) (size 0.6) (drill 0.3) (layers "F.Cu" "B.Cu") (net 11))
 (via (at 79.6544 63.0428) (size 0.6) (drill 0.3) (layers "F.Cu" "B.Cu") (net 11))
 (via (at 68.9864 112.4712) (size 0.6) (drill 0.3) (layers "F.Cu" "B.Cu") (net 11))
 (segment (start 71.5806 105.273) (end 71.5806 103.8894) (width 0.2) (layer "B.Cu") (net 11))
 (segment (start 68.9806 105.273) (end 68.9806 103.8918) (width 0.2) (layer "B.Cu") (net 11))
 (segment (start 67.6806 103.8964) (end 67.691 103.886) (width 0.2) (layer "B.Cu") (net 11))
 (segment (start 72.8806 110.998) (end 72.8806 112.4792) (width 0.2) (layer "B.Cu") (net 11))
 (segment (start 58.043 56.257) (end 58.039 56.261) (width 0.2) (layer "B.Cu") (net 11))
 (segment (start 79.6467 62.0054) (end 79.6467 63.0351) (width 0.2) (layer "B.Cu") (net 11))
 (segment (start 70.2806 105.273) (end 70.2806 103.8872) (width 0.2) (layer "B.Cu") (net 11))
 (segment (start 58.4966 116.1803) (end 58.4966 118.5414) (width 0.2) (layer "B.Cu") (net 11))
 (segment (start 68.9806 103.8918) (end 68.9864 103.886) (width 0.2) (layer "B.Cu") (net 11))
 (segment (start 70.2806 112.4446) (end 70.2818 112.4458) (width 0.2) (layer "B.Cu") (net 11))
 (segment (start 72.8806 112.4792) (end 72.898 112.4966) (width 0.2) (layer "B.Cu") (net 11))
 (segment (start 58.4966 118.5414) (end 58.4962 118.5418) (width 0.2) (layer "B.Cu") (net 11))
 (segment (start 69.6306 105.273) (end 69.6306 103.8952) (width 0.2) (layer "B.Cu") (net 11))
 (segment (start 70.2806 110.998) (end 70.2806 112.4446) (width 0.2) (layer "B.Cu") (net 11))
 (segment (start 67.691 112.5728) (end 67.6806 112.4354) (width 0.2) (layer "B.Cu") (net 11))
 (segment (start 70.9306 103.8976) (end 70.9422 103.886) (width 0.2) (layer "B.Cu") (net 11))
 (segment (start 59.8247 56.257) (end 58.043 56.257) (width 0.2) (layer "B.Cu") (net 11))
 (segment (start 69.6306 103.8952) (end 69.6214 103.886) (width 0.2) (layer "B.Cu") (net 11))
 (segment (start 67.6806 112.4354) (end 67.6806 110.998) (width 0.2) (layer "B.Cu") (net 11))
 (segment (start 70.9306 105.273) (end 70.9306 103.8976) (width 0.2) (layer "B.Cu") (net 11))
 (segment (start 67.0306 110.998) (end 67.0306 112.522) (width 0.2) (layer "B.Cu") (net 11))
 (segment (start 67.6806 105.273) (end 67.6806 103.8964) (width 0.2) (layer "B.Cu") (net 11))
 (segment (start 68.9806 110.998) (end 68.9806 112.4654) (width 0.2) (layer "B.Cu") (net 11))
 (segment (start 79.6467 63.0351) (end 79.6544 63.0428) (width 0.2) (layer "B.Cu") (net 11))
 (segment (start 71.5806 103.8894) (end 71.5772 103.886) (width 0.2) (layer "B.Cu") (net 11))
 (segment (start 68.9806 112.4654) (end 68.9864 112.4712) (width 0.2) (layer "B.Cu") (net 11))
 (segment (start 55.245 59.2328) (end 55.245 60.833) (width 0.2) (layer "B.Cu") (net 18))
 (segment (start 55.245 60.833) (end 53.594 62.484) (width 0.2) (layer "B.Cu") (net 18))
 (segment (start 56.2708 58.207) (end 55.245 59.2328) (width 0.2) (layer "B.Cu") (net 18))
 (segment (start 59.8247 58.207) (end 56.2708 58.207) (width 0.2) (layer "B.Cu") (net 18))
 (segment (start 57.7348 60.807) (end 57.4294 61.1124) (width 0.2) (layer "B.Cu") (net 14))
 (segment (start 57.4294 61.1124) (end 57.4294 68.8086) (width 0.2) (layer "B.Cu") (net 14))
 (segment (start 57.4294 68.8086) (end 53.594 72.644) (width 0.2) (layer "B.Cu") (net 14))
 (segment (start 59.8247 60.807) (end 57.7348 60.807) (width 0.2) (layer "B.Cu") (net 14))
 (segment (start 53.594 57.404) (end 54.091 56.907) (width 0.2) (layer "B.Cu") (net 20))
 (segment (start 54.091 56.907) (end 59.8247 56.907) (width 0.2) (layer "B.Cu") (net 20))
 (segment (start 59.8247 60.157) (end 57.2926 60.157) (width 0.2) (layer "B.Cu") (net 15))
 (segment (start 57.2926 60.157) (end 56.9976 60.452) (width 0.2) (layer "B.Cu") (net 15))
 (segment (start 56.9976 60.452) (end 56.9976 66.7004) (width 0.2) (layer "B.Cu") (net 15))
 (segment (start 56.9976 66.7004) (end 53.594 70.104) (width 0.2) (layer "B.Cu") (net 15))
 (segment (start 58.0192 61.457) (end 57.8304 61.6458) (width 0.2) (layer "B.Cu") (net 13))
 (segment (start 59.8247 61.457) (end 58.0192 61.457) (width 0.2) (layer "B.Cu") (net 13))
 (segment (start 57.8304 70.9476) (end 53.594 75.184) (width 0.2) (layer "B.Cu") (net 13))
 (segment (start 57.8304 61.6458) (end 57.8304 70.9476) (width 0.2) (layer "B.Cu") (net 13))
 (segment (start 57.0282 59.507) (end 56.388 60.1472) (width 0.2) (layer "B.Cu") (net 16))
 (segment (start 59.8247 59.507) (end 57.0282 59.507) (width 0.2) (layer "B.Cu") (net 16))
 (segment (start 56.388 60.1472) (end 56.388 64.77) (width 0.2) (layer "B.Cu") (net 16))
 (segment (start 56.388 64.77) (end 53.594 67.564) (width 0.2) (layer "B.Cu") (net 16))
 (segment (start 59.8045 58.8772) (end 56.6928 58.8772) (width 0.2) (layer "B.Cu") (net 17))
 (segment (start 55.8292 59.7408) (end 55.8292 62.7888) (width 0.2) (layer "B.Cu") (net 17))
 (segment (start 55.8292 62.7888) (end 53.594 65.024) (width 0.2) (layer "B.Cu") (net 17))
 (segment (start 59.8247 58.857) (end 59.8045 58.8772) (width 0.2) (layer "B.Cu") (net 17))
 (segment (start 56.6928 58.8772) (end 55.8292 59.7408) (width 0.2) (layer "B.Cu") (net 17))
 (segment (start 84.328 60.706) (end 84.328 59.0296) (width 0.2) (layer "B.Cu") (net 6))
 (segment (start 84.328 59.0296) (end 83.4038 58.1054) (width 0.2) (layer "B.Cu") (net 6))
 (segment (start 83.4038 58.1054) (end 79.6467 58.1054) (width 0.2) (layer "B.Cu") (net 6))
 (segment (start 86.106 62.484) (end 84.328 60.706) (width 0.2) (layer "B.Cu") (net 6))
 (segment (start 83.0634 67.0614) (end 86.106 70.104) (width 0.2) (layer "B.Cu") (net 3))
 (segment (start 82.6922 60.0554) (end 83.0634 60.4266) (width 0.2) (layer "B.Cu") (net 3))
 (segment (start 79.6467 60.0554) (end 82.6922 60.0554) (width 0.2) (layer "B.Cu") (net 3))
 (segment (start 83.0634 60.4266) (end 83.0634 67.0614) (width 0.2) (layer "B.Cu") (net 3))
 (segment (start 79.6467 61.3554) (end 81.777 61.3554) (width 0.2) (layer "B.Cu") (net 1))
 (segment (start 82.2198 71.2978) (end 86.106 75.184) (width 0.2) (layer "B.Cu") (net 1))
 (segment (start 81.777 61.3554) (end 82.2198 61.7982) (width 0.2) (layer "B.Cu") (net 1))
 (segment (start 82.2198 61.7982) (end 82.2198 71.2978) (width 0.2) (layer "B.Cu") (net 1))
 (segment (start 83.4644 59.6646) (end 83.2052 59.4054) (width 0.2) (layer "B.Cu") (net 4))
 (segment (start 83.2052 59.4054) (end 79.6467 59.4054) (width 0.2) (layer "B.Cu") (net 4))
 (segment (start 83.4644 64.9224) (end 83.4644 59.6646) (width 0.2) (layer "B.Cu") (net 4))
 (segment (start 86.106 67.564) (end 83.4644 64.9224) (width 0.2) (layer "B.Cu") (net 4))
 (segment (start 85.5074 56.8054) (end 86.106 57.404) (width 0.2) (layer "B.Cu") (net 8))
 (segment (start 79.6467 56.8054) (end 85.5074 56.8054) (width 0.2) (layer "B.Cu") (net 8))
 (segment (start 83.6174 57.4554) (end 79.6467 57.4554) (width 0.2) (layer "B.Cu") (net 7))
 (segment (start 86.106 59.944) (end 83.6174 57.4554) (width 0.2) (layer "B.Cu") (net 7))
 (segment (start 86.106 65.024) (end 83.8962 62.8142) (width 0.2) (layer "B.Cu") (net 5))
 (segment (start 83.3934 58.7554) (end 79.6467 58.7554) (width 0.2) (layer "B.Cu") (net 5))
 (segment (start 83.8962 62.8142) (end 83.8962 59.2582) (width 0.2) (layer "B.Cu") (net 5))
 (segment (start 83.8962 59.2582) (end 83.3934 58.7554) (width 0.2) (layer "B.Cu") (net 5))
 (segment (start 82.2192 60.7054) (end 79.6467 60.7054) (width 0.2) (layer "B.Cu") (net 2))
 (segment (start 82.6262 69.1642) (end 82.6262 61.1124) (width 0.2) (layer "B.Cu") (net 2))
 (segment (start 82.6262 61.1124) (end 82.2192 60.7054) (width 0.2) (layer "B.Cu") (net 2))
 (segment (start 86.106 72.644) (end 82.6262 69.1642) (width 0.2) (layer "B.Cu") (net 2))
 (segment (start 71.39463 109.9595) (end 72.2306 109.12353) (width 0.2) (layer "B.Cu") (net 29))
 (segment (start 72.2306 105.273) (end 72.2306 64.5852) (width 0.2) (layer "B.Cu") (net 29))
 (segment (start 72.2306 109.12353) (end 72.2306 105.273) (width 0.2) (layer "B.Cu") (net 29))
 (segment (start 67.6004 61.457) (end 68.7324 60.325) (width 0.2) (layer "B.Cu") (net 29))
 (segment (start 69.6722 59.3852) (end 69.8881 59.1693) (width 0.2) (layer "B.Cu") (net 29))
 (segment (start 65.5497 61.457) (end 67.6004 61.457) (width 0.2) (layer "B.Cu") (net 29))
 (segment (start 62.6847 109.9595) (end 71.39463 109.9595) (width 0.2) (layer "B.Cu") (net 29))
 (segment (start 61.0366 111.6076) (end 62.6847 109.9595) (width 0.2) (layer "B.Cu") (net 29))
 (segment (start 68.7324 61.087) (end 68.7324 60.325) (width 0.2) (layer "B.Cu") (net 29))
 (segment (start 68.7324 60.325) (end 69.6722 59.3852) (width 0.2) (layer "B.Cu") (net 29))
 (segment (start 69.8881 59.1693) (end 72.252 56.8054) (width 0.2) (layer "B.Cu") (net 29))
 (segment (start 72.252 56.8054) (end 73.9217 56.8054) (width 0.2) (layer "B.Cu") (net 29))
 (segment (start 72.2306 64.5852) (end 68.7324 61.087) (width 0.2) (layer "B.Cu") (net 29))
 (via (at 67.1836 60.807) (size 0.6) (drill 0.3) (layers "F.Cu" "B.Cu") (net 28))
 (segment (start 65.5497 60.807) (end 67.1836 60.807) (width 0.2) (layer "B.Cu") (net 28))
 (via (at 63.8708 58.857) (size 0.6) (drill 0.3) (layers "F.Cu" "B.Cu") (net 25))
 (segment (start 65.5497 58.857) (end 63.8708 58.857) (width 0.2) (layer "B.Cu") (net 25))
 (via (at 63.8908 60.157) (size 0.6) (drill 0.3) (layers "F.Cu" "B.Cu") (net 27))
 (segment (start 65.5497 60.157) (end 63.8908 60.157) (width 0.2) (layer "B.Cu") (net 27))
 (via (at 67.2136 59.507) (size 0.6) (drill 0.3) (layers "F.Cu" "B.Cu") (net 26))
 (segment (start 65.5497 59.507) (end 67.2136 59.507) (width 0.2) (layer "B.Cu") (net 26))
 (via (at 75.6118 62.0054) (size 0.6) (drill 0.3) (layers "F.Cu" "B.Cu") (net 30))
 (segment (start 73.9217 62.0054) (end 75.6118 62.0054) (width 0.2) (layer "B.Cu") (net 30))
 (via (at 72.3802 60.0554) (size 0.6) (drill 0.3) (layers "F.Cu" "B.Cu") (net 33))
 (segment (start 73.9217 60.0554) (end 72.3802 60.0554) (width 0.2) (layer "B.Cu") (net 33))
 (via (at 72.461 58.7554) (size 0.6) (drill 0.3) (layers "F.Cu" "B.Cu") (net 35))
 (segment (start 73.9217 58.7554) (end 72.461 58.7554) (width 0.2) (layer "B.Cu") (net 35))
 (via (at 72.4662 61.3664) (size 0.6) (drill 0.3) (layers "F.Cu" "B.Cu") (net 31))
 (segment (start 72.4772 61.3554) (end 72.4662 61.3664) (width 0.2) (layer "B.Cu") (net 31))
 (segment (start 73.9217 61.3554) (end 72.4772 61.3554) (width 0.2) (layer "B.Cu") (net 31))
 (via (at 75.4888 59.4106) (size 0.6) (drill 0.3) (layers "F.Cu" "B.Cu") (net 34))
 (segment (start 73.9217 59.4054) (end 75.3058 59.4054) (width 0.2) (layer "B.Cu") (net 34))
 (segment (start 75.3058 59.4054) (end 75.4836 59.4054) (width 0.2) (layer "B.Cu") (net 34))
 (segment (start 75.4836 59.4054) (end 75.4888 59.4106) (width 0.2) (layer "B.Cu") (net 34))
 (via (at 75.4536 58.1054) (size 0.6) (drill 0.3) (layers "F.Cu" "B.Cu") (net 36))
 (segment (start 73.9217 58.1054) (end 75.4536 58.1054) (width 0.2) (layer "B.Cu") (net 36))
 (via (at 75.565 60.706) (size 0.6) (drill 0.3) (layers "F.Cu" "B.Cu") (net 32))
 (segment (start 73.9217 60.7054) (end 75.337 60.7054) (width 0.2) (layer "B.Cu") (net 32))
 (segment (start 75.3376 60.706) (end 75.565 60.706) (width 0.2) (layer "B.Cu") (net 32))
 (segment (start 75.337 60.7054) (end 75.3376 60.706) (width 0.2) (layer "B.Cu") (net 32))
 (segment (start 63.496987 120.901587) (end 63.496987 118.880687) (width 0.2) (layer "B.Cu") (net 10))
 (segment (start 60.3875 113.8803) (end 60.4008 113.8936) (width 0.2) (layer "B.Cu") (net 10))
 (segment (start 58.4966 113.8803) (end 60.3875 113.8803) (width 0.2) (layer "B.Cu") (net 10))
 (segment (start 63.496987 118.880687) (end 58.4966 113.8803) (width 0.2) (layer "B.Cu") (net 10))
 (segment (start 58.4966 111.5803) (end 60.3693 111.5803) (width 0.2) (layer "B.Cu") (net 9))
 (segment (start 60.3693 111.5803) (end 60.3966 111.6076) (width 0.2) (layer "B.Cu") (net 9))
 (via (at 72.4662 57.4548) (size 0.6) (drill 0.3) (layers "F.Cu" "B.Cu") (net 37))
 (segment (start 73.9217 57.4554) (end 72.4668 57.4554) (width 0.2) (layer "B.Cu") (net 37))
 (segment (start 72.4668 57.4554) (end 72.4662 57.4548) (width 0.2) (layer "B.Cu") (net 37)))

